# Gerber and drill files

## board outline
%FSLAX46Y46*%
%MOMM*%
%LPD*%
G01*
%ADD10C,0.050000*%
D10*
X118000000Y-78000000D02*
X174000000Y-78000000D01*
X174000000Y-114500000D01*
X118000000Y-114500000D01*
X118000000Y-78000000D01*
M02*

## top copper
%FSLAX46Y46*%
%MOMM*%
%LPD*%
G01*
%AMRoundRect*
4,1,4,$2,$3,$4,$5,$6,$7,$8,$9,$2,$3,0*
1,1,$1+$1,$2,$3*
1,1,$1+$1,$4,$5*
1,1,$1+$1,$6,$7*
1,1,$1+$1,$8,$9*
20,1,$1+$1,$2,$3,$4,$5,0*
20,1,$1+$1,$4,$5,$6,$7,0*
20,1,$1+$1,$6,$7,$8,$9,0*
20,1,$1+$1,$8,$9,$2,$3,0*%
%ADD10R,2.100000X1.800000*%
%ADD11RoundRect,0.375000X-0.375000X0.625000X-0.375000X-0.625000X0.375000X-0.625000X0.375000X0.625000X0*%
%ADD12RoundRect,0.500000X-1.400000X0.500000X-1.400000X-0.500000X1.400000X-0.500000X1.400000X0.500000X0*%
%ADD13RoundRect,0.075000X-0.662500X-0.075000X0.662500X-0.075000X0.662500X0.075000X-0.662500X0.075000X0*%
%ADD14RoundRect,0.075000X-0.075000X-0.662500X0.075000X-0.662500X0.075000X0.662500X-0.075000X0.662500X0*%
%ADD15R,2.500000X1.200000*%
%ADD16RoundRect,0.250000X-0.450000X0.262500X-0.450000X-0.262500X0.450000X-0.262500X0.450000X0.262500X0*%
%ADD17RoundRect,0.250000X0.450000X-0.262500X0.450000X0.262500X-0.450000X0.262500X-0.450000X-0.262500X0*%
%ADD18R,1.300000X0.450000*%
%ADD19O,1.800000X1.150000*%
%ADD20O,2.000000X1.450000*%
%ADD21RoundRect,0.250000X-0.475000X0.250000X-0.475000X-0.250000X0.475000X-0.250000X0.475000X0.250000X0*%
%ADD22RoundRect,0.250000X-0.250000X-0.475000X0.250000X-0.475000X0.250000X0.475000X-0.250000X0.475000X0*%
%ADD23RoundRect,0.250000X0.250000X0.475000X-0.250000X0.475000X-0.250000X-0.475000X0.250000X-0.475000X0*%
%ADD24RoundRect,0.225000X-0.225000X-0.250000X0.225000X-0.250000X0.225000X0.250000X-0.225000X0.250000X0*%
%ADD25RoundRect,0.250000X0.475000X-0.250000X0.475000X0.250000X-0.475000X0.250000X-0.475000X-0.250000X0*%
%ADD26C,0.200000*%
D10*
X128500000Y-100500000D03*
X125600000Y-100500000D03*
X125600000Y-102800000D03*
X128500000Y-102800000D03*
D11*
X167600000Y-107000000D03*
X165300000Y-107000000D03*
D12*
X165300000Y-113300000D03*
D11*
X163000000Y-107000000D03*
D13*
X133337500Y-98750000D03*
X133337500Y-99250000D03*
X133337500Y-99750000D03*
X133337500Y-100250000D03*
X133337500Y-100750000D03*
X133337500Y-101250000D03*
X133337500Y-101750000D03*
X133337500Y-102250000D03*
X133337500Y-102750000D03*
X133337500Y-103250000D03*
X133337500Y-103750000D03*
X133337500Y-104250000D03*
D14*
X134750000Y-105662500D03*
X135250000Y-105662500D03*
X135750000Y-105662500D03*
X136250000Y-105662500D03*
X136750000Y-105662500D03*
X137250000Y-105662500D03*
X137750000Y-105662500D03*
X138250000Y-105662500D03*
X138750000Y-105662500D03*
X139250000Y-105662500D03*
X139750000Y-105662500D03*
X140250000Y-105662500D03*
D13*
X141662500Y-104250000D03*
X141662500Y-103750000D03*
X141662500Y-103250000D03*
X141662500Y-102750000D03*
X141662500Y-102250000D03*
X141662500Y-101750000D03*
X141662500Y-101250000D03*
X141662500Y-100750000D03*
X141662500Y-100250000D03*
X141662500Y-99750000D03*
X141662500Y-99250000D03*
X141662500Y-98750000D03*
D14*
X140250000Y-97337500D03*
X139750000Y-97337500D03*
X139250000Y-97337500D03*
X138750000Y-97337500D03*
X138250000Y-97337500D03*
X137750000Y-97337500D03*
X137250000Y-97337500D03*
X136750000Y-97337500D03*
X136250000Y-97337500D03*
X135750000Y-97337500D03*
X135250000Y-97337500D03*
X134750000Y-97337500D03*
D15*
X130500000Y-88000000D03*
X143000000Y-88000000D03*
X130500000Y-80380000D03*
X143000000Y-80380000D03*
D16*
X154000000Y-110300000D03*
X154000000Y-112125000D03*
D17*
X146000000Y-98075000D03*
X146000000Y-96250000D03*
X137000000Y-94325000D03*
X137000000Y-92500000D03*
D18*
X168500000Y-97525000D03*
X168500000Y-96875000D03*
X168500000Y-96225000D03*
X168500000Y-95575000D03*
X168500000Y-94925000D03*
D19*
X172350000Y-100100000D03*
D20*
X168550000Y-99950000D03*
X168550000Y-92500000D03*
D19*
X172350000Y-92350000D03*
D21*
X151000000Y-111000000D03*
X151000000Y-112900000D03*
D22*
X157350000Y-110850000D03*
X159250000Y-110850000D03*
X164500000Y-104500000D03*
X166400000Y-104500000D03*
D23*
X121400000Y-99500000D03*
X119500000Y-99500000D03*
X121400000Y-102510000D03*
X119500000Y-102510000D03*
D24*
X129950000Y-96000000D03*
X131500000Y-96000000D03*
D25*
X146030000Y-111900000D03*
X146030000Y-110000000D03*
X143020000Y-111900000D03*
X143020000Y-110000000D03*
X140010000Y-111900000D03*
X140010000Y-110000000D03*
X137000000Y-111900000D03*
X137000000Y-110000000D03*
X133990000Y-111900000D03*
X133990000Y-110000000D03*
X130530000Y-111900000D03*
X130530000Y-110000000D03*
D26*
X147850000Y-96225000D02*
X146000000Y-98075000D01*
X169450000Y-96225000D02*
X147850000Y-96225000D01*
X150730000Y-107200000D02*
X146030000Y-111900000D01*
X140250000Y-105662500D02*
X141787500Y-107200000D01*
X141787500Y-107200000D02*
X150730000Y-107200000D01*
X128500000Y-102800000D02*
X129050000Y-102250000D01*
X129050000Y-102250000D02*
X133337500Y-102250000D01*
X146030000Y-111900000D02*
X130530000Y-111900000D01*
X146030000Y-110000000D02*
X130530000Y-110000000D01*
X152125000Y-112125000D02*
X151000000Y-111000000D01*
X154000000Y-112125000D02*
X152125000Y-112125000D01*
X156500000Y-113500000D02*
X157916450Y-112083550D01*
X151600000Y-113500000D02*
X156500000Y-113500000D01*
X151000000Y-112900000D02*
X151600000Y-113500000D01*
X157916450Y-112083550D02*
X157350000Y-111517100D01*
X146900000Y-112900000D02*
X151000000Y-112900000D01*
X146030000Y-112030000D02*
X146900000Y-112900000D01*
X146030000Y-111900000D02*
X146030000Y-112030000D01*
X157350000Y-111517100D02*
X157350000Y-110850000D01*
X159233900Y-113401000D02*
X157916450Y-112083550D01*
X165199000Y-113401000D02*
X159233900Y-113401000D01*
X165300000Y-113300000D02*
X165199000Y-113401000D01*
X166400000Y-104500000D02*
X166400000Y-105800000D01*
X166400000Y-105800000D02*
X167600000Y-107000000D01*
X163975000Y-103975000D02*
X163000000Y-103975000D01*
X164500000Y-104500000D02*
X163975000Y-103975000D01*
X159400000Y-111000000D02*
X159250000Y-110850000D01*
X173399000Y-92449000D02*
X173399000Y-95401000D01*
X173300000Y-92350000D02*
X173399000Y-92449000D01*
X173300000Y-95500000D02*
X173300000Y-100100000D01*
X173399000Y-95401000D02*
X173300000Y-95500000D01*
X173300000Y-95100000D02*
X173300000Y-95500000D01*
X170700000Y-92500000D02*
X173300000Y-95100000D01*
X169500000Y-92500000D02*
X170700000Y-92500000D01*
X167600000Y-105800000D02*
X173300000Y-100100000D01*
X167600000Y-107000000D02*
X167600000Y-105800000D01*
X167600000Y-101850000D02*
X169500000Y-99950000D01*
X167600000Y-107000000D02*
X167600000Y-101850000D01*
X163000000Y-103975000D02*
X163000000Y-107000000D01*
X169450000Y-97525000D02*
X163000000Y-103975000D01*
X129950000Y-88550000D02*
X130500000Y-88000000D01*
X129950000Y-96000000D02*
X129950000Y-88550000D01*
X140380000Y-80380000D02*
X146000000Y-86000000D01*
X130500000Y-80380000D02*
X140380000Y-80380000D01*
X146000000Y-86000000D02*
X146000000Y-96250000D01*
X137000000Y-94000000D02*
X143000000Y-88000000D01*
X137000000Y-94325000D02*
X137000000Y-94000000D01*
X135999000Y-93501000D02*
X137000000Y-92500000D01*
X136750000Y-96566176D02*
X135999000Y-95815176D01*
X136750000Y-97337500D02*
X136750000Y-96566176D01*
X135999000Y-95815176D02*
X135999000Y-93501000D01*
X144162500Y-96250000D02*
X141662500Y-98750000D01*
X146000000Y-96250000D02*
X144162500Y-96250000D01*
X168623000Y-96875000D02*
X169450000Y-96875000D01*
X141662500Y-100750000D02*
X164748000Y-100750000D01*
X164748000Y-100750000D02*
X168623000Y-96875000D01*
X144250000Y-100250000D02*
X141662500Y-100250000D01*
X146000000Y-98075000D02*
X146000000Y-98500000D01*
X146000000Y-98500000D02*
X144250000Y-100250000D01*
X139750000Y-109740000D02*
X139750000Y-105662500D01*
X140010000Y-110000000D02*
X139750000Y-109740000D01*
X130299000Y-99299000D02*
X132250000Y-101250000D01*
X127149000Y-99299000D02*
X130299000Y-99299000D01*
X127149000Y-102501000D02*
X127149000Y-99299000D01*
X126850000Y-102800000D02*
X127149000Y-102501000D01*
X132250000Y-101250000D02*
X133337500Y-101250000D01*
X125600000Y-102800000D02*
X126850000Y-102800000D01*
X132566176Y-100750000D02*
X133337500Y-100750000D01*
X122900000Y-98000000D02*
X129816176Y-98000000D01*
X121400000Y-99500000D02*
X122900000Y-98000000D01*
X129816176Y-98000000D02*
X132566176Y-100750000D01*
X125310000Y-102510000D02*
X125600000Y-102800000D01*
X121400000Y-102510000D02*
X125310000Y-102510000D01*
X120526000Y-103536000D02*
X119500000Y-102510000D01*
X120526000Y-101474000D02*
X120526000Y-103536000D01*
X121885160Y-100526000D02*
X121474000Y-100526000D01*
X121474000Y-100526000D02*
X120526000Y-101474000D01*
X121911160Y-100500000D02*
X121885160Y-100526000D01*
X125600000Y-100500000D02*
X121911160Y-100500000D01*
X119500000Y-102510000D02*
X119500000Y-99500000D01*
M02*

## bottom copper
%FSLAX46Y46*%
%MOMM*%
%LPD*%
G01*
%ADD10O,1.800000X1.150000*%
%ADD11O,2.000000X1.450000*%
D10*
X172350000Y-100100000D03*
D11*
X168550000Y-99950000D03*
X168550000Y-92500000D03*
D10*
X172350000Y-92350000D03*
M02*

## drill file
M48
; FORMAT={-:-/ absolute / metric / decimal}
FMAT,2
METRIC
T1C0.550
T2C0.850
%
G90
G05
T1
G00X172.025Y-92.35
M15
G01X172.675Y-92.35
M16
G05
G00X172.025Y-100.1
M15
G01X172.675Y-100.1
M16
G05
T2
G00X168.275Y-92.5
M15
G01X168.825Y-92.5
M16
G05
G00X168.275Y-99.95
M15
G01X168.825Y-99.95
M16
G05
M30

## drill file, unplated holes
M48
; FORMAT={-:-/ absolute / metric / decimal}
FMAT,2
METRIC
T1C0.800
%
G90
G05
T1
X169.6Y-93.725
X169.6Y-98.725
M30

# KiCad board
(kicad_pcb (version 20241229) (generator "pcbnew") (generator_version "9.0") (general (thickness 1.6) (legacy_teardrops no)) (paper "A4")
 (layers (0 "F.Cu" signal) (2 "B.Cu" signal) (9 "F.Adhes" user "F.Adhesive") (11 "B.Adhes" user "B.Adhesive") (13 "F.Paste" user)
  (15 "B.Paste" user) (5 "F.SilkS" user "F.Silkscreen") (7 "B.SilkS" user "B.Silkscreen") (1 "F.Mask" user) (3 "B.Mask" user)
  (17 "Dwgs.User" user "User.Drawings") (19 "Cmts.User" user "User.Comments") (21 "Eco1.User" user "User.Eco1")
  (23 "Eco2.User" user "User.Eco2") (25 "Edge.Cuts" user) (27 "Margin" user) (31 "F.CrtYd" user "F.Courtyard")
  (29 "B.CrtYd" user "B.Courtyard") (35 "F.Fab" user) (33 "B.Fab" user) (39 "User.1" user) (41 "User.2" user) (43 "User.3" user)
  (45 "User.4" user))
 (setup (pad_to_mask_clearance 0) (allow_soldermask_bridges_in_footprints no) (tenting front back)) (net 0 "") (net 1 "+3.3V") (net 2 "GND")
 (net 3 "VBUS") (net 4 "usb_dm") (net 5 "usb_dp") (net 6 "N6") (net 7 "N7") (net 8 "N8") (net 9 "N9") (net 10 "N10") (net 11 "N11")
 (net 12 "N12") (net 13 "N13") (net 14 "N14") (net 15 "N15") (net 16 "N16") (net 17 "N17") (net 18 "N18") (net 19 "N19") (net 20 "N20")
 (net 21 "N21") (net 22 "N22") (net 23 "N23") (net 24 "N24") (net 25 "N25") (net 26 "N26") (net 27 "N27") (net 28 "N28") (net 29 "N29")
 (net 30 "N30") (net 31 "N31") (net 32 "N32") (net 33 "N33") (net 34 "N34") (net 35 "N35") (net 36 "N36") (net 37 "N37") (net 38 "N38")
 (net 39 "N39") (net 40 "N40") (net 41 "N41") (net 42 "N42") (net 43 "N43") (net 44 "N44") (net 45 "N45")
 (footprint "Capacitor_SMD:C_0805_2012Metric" (layer "F.Cu") (at 133.99 110.95 90)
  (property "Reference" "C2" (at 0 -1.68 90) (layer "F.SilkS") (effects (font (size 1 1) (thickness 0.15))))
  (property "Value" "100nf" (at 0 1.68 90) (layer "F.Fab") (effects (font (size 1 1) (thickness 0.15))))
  (pad "1" smd roundrect (at -0.95 0 90) (size 1 1.45) (layers "F.Cu" "F.Mask" "F.Paste") (roundrect_rratio 0.25) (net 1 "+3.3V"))
  (pad "2" smd roundrect (at 0.95 0 90) (size 1 1.45) (layers "F.Cu" "F.Mask" "F.Paste") (roundrect_rratio 0.25) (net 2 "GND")))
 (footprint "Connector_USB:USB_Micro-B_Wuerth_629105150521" (layer "F.Cu") (at 170.4 96.225 90)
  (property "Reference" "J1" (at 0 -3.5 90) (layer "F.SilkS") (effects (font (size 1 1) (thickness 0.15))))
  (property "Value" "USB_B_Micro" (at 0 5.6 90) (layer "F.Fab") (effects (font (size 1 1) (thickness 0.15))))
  (pad "" np_thru_hole oval (at -2.5 -0.8 90) (size 0.8 0.8) (drill 0.8) (layers "*.Cu" "*.Mask"))
  (pad "" np_thru_hole oval (at 2.5 -0.8 90) (size 0.8 0.8) (drill 0.8) (layers "*.Cu" "*.Mask"))
  (pad "1" smd rect (at -1.3 -1.9 90) (size 0.45 1.3) (layers "F.Cu" "F.Mask" "F.Paste") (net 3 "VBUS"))
  (pad "2" smd rect (at -0.65 -1.9 90) (size 0.45 1.3) (layers "F.Cu" "F.Mask" "F.Paste") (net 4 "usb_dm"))
  (pad "3" smd rect (at 0 -1.9 90) (size 0.45 1.3) (layers "F.Cu" "F.Mask" "F.Paste") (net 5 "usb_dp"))
  (pad "4" smd rect (at 0.65 -1.9 90) (size 0.45 1.3) (layers "F.Cu" "F.Mask" "F.Paste") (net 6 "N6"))
  (pad "5" smd rect (at 1.3 -1.9 90) (size 0.45 1.3) (layers "F.Cu" "F.Mask" "F.Paste") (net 2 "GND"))
  (pad "6" thru_hole oval (at -3.875 1.95 90) (size 1.15 1.8) (drill oval 0.55 1.2) (layers "*.Cu" "*.Mask") (remove_unused_layers no)
   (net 2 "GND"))
  (pad "6" thru_hole oval (at -3.725 -1.85 90) (size 1.45 2) (drill oval 0.85 1.4) (layers "*.Cu" "*.Mask") (remove_unused_layers no)
   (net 2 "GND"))
  (pad "6" thru_hole oval (at 3.725 -1.85 90) (size 1.45 2) (drill oval 0.85 1.4) (layers "*.Cu" "*.Mask") (remove_unused_layers no)
   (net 2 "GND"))
  (pad "6" thru_hole oval (at 3.875 1.95 90) (size 1.15 1.8) (drill oval 0.55 1.2) (layers "*.Cu" "*.Mask") (remove_unused_layers no)
   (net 2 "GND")))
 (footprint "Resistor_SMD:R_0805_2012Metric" (layer "F.Cu") (at 137 93.4125 90)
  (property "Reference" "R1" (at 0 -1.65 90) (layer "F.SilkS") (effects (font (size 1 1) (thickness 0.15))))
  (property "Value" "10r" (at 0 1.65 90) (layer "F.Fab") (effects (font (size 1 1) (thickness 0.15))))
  (pad "1" smd roundrect (at -0.9125 0 90) (size 1.025 1.4) (layers "F.Cu" "F.Mask" "F.Paste") (roundrect_rratio 0.243902) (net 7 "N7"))
  (pad "2" smd roundrect (at 0.9125 0 90) (size 1.025 1.4) (layers "F.Cu" "F.Mask" "F.Paste") (roundrect_rratio 0.243902) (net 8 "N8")))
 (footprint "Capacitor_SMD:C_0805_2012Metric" (layer "F.Cu") (at 143.02 110.95 90)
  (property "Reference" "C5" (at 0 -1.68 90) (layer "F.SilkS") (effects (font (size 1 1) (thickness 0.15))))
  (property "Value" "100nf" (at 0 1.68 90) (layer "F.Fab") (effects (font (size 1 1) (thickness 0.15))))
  (pad "1" smd roundrect (at -0.95 0 90) (size 1 1.45) (layers "F.Cu" "F.Mask" "F.Paste") (roundrect_rratio 0.25) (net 1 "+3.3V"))
  (pad "2" smd roundrect (at 0.95 0 90) (size 1 1.45) (layers "F.Cu" "F.Mask" "F.Paste") (roundrect_rratio 0.25) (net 2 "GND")))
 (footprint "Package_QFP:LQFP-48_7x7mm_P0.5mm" (layer "F.Cu") (at 137.5 101.5)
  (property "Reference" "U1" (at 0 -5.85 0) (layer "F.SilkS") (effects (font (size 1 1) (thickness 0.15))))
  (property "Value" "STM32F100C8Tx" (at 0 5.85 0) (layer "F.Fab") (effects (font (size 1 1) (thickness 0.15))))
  (pad "1" smd roundrect (at -4.1625 -2.75) (size 1.475 0.3) (layers "F.Cu" "F.Mask" "F.Paste") (roundrect_rratio 0.25) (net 1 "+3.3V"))
  (pad "2" smd roundrect (at -4.1625 -2.25) (size 1.475 0.3) (layers "F.Cu" "F.Mask" "F.Paste") (roundrect_rratio 0.25) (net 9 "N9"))
  (pad "3" smd roundrect (at -4.1625 -1.75) (size 1.475 0.3) (layers "F.Cu" "F.Mask" "F.Paste") (roundrect_rratio 0.25) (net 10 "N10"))
  (pad "4" smd roundrect (at -4.1625 -1.25) (size 1.475 0.3) (layers "F.Cu" "F.Mask" "F.Paste") (roundrect_rratio 0.25) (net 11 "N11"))
  (pad "5" smd roundrect (at -4.1625 -0.75) (size 1.475 0.3) (layers "F.Cu" "F.Mask" "F.Paste") (roundrect_rratio 0.25) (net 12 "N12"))
  (pad "6" smd roundrect (at -4.1625 -0.25) (size 1.475 0.3) (layers "F.Cu" "F.Mask" "F.Paste") (roundrect_rratio 0.25) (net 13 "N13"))
  (pad "7" smd roundrect (at -4.1625 0.25) (size 1.475 0.3) (layers "F.Cu" "F.Mask" "F.Paste") (roundrect_rratio 0.25) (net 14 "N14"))
  (pad "8" smd roundrect (at -4.1625 0.75) (size 1.475 0.3) (layers "F.Cu" "F.Mask" "F.Paste") (roundrect_rratio 0.25) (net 2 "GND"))
  (pad "9" smd roundrect (at -4.1625 1.25) (size 1.475 0.3) (layers "F.Cu" "F.Mask" "F.Paste") (roundrect_rratio 0.25) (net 1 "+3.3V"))
  (pad "10" smd roundrect (at -4.1625 1.75) (size 1.475 0.3) (layers "F.Cu" "F.Mask" "F.Paste") (roundrect_rratio 0.25) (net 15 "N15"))
  (pad "11" smd roundrect (at -4.1625 2.25) (size 1.475 0.3) (layers "F.Cu" "F.Mask" "F.Paste") (roundrect_rratio 0.25) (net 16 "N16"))
  (pad "12" smd roundrect (at -4.1625 2.75) (size 1.475 0.3) (layers "F.Cu" "F.Mask" "F.Paste") (roundrect_rratio 0.25) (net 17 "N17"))
  (pad "13" smd roundrect (at -2.75 4.1625) (size 0.3 1.475) (layers "F.Cu" "F.Mask" "F.Paste") (roundrect_rratio 0.25) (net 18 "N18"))
  (pad "14" smd roundrect (at -2.25 4.1625) (size 0.3 1.475) (layers "F.Cu" "F.Mask" "F.Paste") (roundrect_rratio 0.25) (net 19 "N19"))
  (pad "15" smd roundrect (at -1.75 4.1625) (size 0.3 1.475) (layers "F.Cu" "F.Mask" "F.Paste") (roundrect_rratio 0.25) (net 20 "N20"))
  (pad "16" smd roundrect (at -1.25 4.1625) (size 0.3 1.475) (layers "F.Cu" "F.Mask" "F.Paste") (roundrect_rratio 0.25) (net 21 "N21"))
  (pad "17" smd roundrect (at -0.75 4.1625) (size 0.3 1.475) (layers "F.Cu" "F.Mask" "F.Paste") (roundrect_rratio 0.25) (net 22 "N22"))
  (pad "18" smd roundrect (at -0.25 4.1625) (size 0.3 1.475) (layers "F.Cu" "F.Mask" "F.Paste") (roundrect_rratio 0.25) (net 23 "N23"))
  (pad "19" smd roundrect (at 0.25 4.1625) (size 0.3 1.475) (layers "F.Cu" "F.Mask" "F.Paste") (roundrect_rratio 0.25) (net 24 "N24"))
  (pad "20" smd roundrect (at 0.75 4.1625) (size 0.3 1.475) (layers "F.Cu" "F.Mask" "F.Paste") (roundrect_rratio 0.25) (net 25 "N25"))
  (pad "21" smd roundrect (at 1.25 4.1625) (size 0.3 1.475) (layers "F.Cu" "F.Mask" "F.Paste") (roundrect_rratio 0.25) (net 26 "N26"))
  (pad "22" smd roundrect (at 1.75 4.1625) (size 0.3 1.475) (layers "F.Cu" "F.Mask" "F.Paste") (roundrect_rratio 0.25) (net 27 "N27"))
  (pad "23" smd roundrect (at 2.25 4.1625) (size 0.3 1.475) (layers "F.Cu" "F.Mask" "F.Paste") (roundrect_rratio 0.25) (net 2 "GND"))
  (pad "24" smd roundrect (at 2.75 4.1625) (size 0.3 1.475) (layers "F.Cu" "F.Mask" "F.Paste") (roundrect_rratio 0.25) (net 1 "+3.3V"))
  (pad "25" smd roundrect (at 4.1625 2.75) (size 1.475 0.3) (layers "F.Cu" "F.Mask" "F.Paste") (roundrect_rratio 0.25) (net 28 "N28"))
  (pad "26" smd roundrect (at 4.1625 2.25) (size 1.475 0.3) (layers "F.Cu" "F.Mask" "F.Paste") (roundrect_rratio 0.25) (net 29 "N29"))
  (pad "27" smd roundrect (at 4.1625 1.75) (size 1.475 0.3) (layers "F.Cu" "F.Mask" "F.Paste") (roundrect_rratio 0.25) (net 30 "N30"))
  (pad "28" smd roundrect (at 4.1625 1.25) (size 1.475 0.3) (layers "F.Cu" "F.Mask" "F.Paste") (roundrect_rratio 0.25) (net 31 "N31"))
  (pad "29" smd roundrect (at 4.1625 0.75) (size 1.475 0.3) (layers "F.Cu" "F.Mask" "F.Paste") (roundrect_rratio 0.25) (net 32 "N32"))
  (pad "30" smd roundrect (at 4.1625 0.25) (size 1.475 0.3) (layers "F.Cu" "F.Mask" "F.Paste") (roundrect_rratio 0.25) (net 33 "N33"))
  (pad "31" smd roundrect (at 4.1625 -0.25) (size 1.475 0.3) (layers "F.Cu" "F.Mask" "F.Paste") (roundrect_rratio 0.25) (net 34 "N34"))
  (pad "32" smd roundrect (at 4.1625 -0.75) (size 1.475 0.3) (layers "F.Cu" "F.Mask" "F.Paste") (roundrect_rratio 0.25) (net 4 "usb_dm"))
  (pad "33" smd roundrect (at 4.1625 -1.25) (size 1.475 0.3) (layers "F.Cu" "F.Mask" "F.Paste") (roundrect_rratio 0.25) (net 5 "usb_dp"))
  (pad "34" smd roundrect (at 4.1625 -1.75) (size 1.475 0.3) (layers "F.Cu" "F.Mask" "F.Paste") (roundrect_rratio 0.25) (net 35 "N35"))
  (pad "35" smd roundrect (at 4.1625 -2.25) (size 1.475 0.3) (layers "F.Cu" "F.Mask" "F.Paste") (roundrect_rratio 0.25) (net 2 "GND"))
  (pad "36" smd roundrect (at 4.1625 -2.75) (size 1.475 0.3) (layers "F.Cu" "F.Mask" "F.Paste") (roundrect_rratio 0.25) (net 1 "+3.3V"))
  (pad "37" smd roundrect (at 2.75 -4.1625) (size 0.3 1.475) (layers "F.Cu" "F.Mask" "F.Paste") (roundrect_rratio 0.25) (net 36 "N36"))
  (pad "38" smd roundrect (at 2.25 -4.1625) (size 0.3 1.475) (layers "F.Cu" "F.Mask" "F.Paste") (roundrect_rratio 0.25) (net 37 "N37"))
  (pad "39" smd roundrect (at 1.75 -4.1625) (size 0.3 1.475) (layers "F.Cu" "F.Mask" "F.Paste") (roundrect_rratio 0.25) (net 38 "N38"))
  (pad "40" smd roundrect (at 1.25 -4.1625) (size 0.3 1.475) (layers "F.Cu" "F.Mask" "F.Paste") (roundrect_rratio 0.25) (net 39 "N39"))
  (pad "41" smd roundrect (at 0.75 -4.1625) (size 0.3 1.475) (layers "F.Cu" "F.Mask" "F.Paste") (roundrect_rratio 0.25) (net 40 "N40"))
  (pad "42" smd roundrect (at 0.25 -4.1625) (size 0.3 1.475) (layers "F.Cu" "F.Mask" "F.Paste") (roundrect_rratio 0.25) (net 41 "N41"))
  (pad "43" smd roundrect (at -0.25 -4.1625) (size 0.3 1.475) (layers "F.Cu" "F.Mask" "F.Paste") (roundrect_rratio 0.25) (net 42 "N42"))
  (pad "44" smd roundrect (at -0.75 -4.1625) (size 0.3 1.475) (layers "F.Cu" "F.Mask" "F.Paste") (roundrect_rratio 0.25) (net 8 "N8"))
  (pad "45" smd roundrect (at -1.25 -4.1625) (size 0.3 1.475) (layers "F.Cu" "F.Mask" "F.Paste") (roundrect_rratio 0.25) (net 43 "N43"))
  (pad "46" smd roundrect (at -1.75 -4.1625) (size 0.3 1.475) (layers "F.Cu" "F.Mask" "F.Paste") (roundrect_rratio 0.25) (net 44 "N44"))
  (pad "47" smd roundrect (at -2.25 -4.1625) (size 0.3 1.475) (layers "F.Cu" "F.Mask" "F.Paste") (roundrect_rratio 0.25) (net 2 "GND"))
  (pad "48" smd roundrect (at -2.75 -4.1625) (size 0.3 1.475) (layers "F.Cu" "F.Mask" "F.Paste") (roundrect_rratio 0.25) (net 1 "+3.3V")))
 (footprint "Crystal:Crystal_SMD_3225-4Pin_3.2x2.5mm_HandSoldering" (layer "F.Cu") (at 127.05 101.65 180)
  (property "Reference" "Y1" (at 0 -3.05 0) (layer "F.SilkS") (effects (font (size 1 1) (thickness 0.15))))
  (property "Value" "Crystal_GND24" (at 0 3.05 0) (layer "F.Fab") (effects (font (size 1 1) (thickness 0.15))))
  (pad "1" smd rect (at -1.45 1.15 180) (size 2.1 1.8) (layers "F.Cu" "F.Mask" "F.Paste") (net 12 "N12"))
  (pad "2" smd rect (at 1.45 1.15 180) (size 2.1 1.8) (layers "F.Cu" "F.Mask" "F.Paste") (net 2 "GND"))
  (pad "3" smd rect (at 1.45 -1.15 180) (size 2.1 1.8) (layers "F.Cu" "F.Mask" "F.Paste") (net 13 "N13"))
  (pad "4" smd rect (at -1.45 -1.15 180) (size 2.1 1.8) (layers "F.Cu" "F.Mask" "F.Paste") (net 2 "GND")))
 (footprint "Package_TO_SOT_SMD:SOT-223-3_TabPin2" (layer "F.Cu") (at 165.3 110.15 -90)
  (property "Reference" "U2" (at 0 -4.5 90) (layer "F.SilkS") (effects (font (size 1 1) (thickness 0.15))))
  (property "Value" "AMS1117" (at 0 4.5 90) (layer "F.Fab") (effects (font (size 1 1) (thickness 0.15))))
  (pad "1" smd roundrect (at -3.15 -2.3 270) (size 2 1.5) (layers "F.Cu" "F.Mask" "F.Paste") (roundrect_rratio 0.25) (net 2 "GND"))
  (pad "2" smd roundrect (at -3.15 0 270) (size 2 1.5) (layers "F.Cu" "F.Mask" "F.Paste") (roundrect_rratio 0.25) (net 1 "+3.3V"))
  (pad "2" smd roundrect (at 3.15 0 270) (size 2 3.8) (layers "F.Cu" "F.Mask" "F.Paste") (roundrect_rratio 0.25) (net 1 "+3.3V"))
  (pad "3" smd roundrect (at -3.15 2.3 270) (size 2 1.5) (layers "F.Cu" "F.Mask" "F.Paste") (roundrect_rratio 0.25) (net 3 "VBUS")))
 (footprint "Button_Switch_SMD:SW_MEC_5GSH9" (layer "F.Cu") (at 136.75 84.19 90)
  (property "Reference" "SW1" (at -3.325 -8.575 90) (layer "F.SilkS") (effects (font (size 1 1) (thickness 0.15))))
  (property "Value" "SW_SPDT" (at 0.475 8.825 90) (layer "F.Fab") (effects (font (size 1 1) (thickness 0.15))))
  (pad "1" smd rect (at -3.81 -6.25 180) (size 2.5 1.2) (layers "F.Cu" "F.Mask" "F.Paste") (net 2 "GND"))
  (pad "2" smd rect (at -3.81 6.25 180) (size 2.5 1.2) (layers "F.Cu" "F.Mask" "F.Paste") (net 7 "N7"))
  (pad "3" smd rect (at 3.81 -6.25 180) (size 2.5 1.2) (layers "F.Cu" "F.Mask" "F.Paste") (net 1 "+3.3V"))
  (pad "4" smd rect (at 3.81 6.25 180) (size 2.5 1.2) (layers "F.Cu" "F.Mask" "F.Paste")))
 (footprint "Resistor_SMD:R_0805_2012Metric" (layer "F.Cu") (at 154 111.2125 -90)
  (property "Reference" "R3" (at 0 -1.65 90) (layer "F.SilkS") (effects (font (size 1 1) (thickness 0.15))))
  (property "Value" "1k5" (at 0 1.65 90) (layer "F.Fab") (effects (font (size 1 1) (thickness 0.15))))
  (pad "1" smd roundrect (at -0.9125 0 270) (size 1.025 1.4) (layers "F.Cu" "F.Mask" "F.Paste") (roundrect_rratio 0.243902) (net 2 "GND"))
  (pad "2" smd roundrect (at 0.9125 0 270) (size 1.025 1.4) (layers "F.Cu" "F.Mask" "F.Paste") (roundrect_rratio 0.243902) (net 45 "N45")))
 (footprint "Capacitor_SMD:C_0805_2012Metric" (layer "F.Cu") (at 140.01 110.95 90)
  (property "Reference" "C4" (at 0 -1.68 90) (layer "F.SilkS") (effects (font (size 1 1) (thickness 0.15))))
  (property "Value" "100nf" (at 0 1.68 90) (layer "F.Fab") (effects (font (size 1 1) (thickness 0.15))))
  (pad "1" smd roundrect (at -0.95 0 90) (size 1 1.45) (layers "F.Cu" "F.Mask" "F.Paste") (roundrect_rratio 0.25) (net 1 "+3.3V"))
  (pad "2" smd roundrect (at 0.95 0 90) (size 1 1.45) (layers "F.Cu" "F.Mask" "F.Paste") (roundrect_rratio 0.25) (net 2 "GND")))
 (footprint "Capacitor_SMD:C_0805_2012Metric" (layer "F.Cu") (at 120.45 102.51 180)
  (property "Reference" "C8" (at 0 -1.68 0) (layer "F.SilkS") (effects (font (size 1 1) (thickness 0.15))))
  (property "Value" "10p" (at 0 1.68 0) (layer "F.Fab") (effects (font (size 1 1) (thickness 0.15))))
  (pad "1" smd roundrect (at -0.95 0 180) (size 1 1.45) (layers "F.Cu" "F.Mask" "F.Paste") (roundrect_rratio 0.25) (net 13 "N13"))
  (pad "2" smd roundrect (at 0.95 0 180) (size 1 1.45) (layers "F.Cu" "F.Mask" "F.Paste") (roundrect_rratio 0.25) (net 2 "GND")))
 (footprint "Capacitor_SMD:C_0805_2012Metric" (layer "F.Cu") (at 151 111.95 -90)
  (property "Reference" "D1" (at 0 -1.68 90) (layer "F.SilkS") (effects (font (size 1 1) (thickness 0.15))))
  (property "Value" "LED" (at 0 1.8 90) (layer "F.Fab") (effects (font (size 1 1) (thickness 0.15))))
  (pad "1" smd roundrect (at -0.95 0 270) (size 1 1.45) (layers "F.Cu" "F.Mask" "F.Paste") (roundrect_rratio 0.25) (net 45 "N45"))
  (pad "2" smd roundrect (at 0.95 0 270) (size 1 1.45) (layers "F.Cu" "F.Mask" "F.Paste") (roundrect_rratio 0.25) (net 1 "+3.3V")))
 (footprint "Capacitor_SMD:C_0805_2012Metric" (layer "F.Cu") (at 165.45 104.5)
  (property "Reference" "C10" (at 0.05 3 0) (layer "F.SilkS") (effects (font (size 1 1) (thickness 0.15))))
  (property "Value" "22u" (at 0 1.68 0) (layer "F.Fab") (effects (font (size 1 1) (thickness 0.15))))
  (pad "1" smd roundrect (at -0.95 0) (size 1 1.45) (layers "F.Cu" "F.Mask" "F.Paste") (roundrect_rratio 0.25) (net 3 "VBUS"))
  (pad "2" smd roundrect (at 0.95 0) (size 1 1.45) (layers "F.Cu" "F.Mask" "F.Paste") (roundrect_rratio 0.25) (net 2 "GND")))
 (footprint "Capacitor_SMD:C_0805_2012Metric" (layer "F.Cu") (at 146.03 110.95 90)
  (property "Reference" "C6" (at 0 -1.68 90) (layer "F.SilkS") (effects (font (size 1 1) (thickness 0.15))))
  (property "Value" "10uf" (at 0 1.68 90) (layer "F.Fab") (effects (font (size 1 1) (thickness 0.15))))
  (pad "1" smd roundrect (at -0.95 0 90) (size 1 1.45) (layers "F.Cu" "F.Mask" "F.Paste") (roundrect_rratio 0.25) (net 1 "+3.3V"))
  (pad "2" smd roundrect (at 0.95 0 90) (size 1 1.45) (layers "F.Cu" "F.Mask" "F.Paste") (roundrect_rratio 0.25) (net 2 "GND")))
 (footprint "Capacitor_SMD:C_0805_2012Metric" (layer "F.Cu") (at 158.3 110.85)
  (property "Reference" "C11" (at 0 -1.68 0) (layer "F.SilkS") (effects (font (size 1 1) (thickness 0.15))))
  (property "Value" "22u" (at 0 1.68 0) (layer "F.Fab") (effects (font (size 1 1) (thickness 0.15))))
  (pad "1" smd roundrect (at -0.95 0) (size 1 1.45) (layers "F.Cu" "F.Mask" "F.Paste") (roundrect_rratio 0.25) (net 1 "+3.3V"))
  (pad "2" smd roundrect (at 0.95 0) (size 1 1.45) (layers "F.Cu" "F.Mask" "F.Paste") (roundrect_rratio 0.25) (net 2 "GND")))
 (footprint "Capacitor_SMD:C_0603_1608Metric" (layer "F.Cu") (at 130.725 96)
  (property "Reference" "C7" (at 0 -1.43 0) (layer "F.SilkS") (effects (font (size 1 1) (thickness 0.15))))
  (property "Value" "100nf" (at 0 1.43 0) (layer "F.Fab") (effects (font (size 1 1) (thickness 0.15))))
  (pad "1" smd roundrect (at -0.775 0) (size 0.9 0.95) (layers "F.Cu" "F.Mask" "F.Paste") (roundrect_rratio 0.25) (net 2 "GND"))
  (pad "2" smd roundrect (at 0.775 0) (size 0.9 0.95) (layers "F.Cu" "F.Mask" "F.Paste") (roundrect_rratio 0.25) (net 14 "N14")))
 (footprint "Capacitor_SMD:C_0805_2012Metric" (layer "F.Cu") (at 120.45 99.5 180)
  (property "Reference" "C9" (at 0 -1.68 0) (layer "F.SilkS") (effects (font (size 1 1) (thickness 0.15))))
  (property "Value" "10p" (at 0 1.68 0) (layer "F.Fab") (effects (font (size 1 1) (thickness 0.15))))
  (pad "1" smd roundrect (at -0.95 0 180) (size 1 1.45) (layers "F.Cu" "F.Mask" "F.Paste") (roundrect_rratio 0.25) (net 12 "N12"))
  (pad "2" smd roundrect (at 0.95 0 180) (size 1 1.45) (layers "F.Cu" "F.Mask" "F.Paste") (roundrect_rratio 0.25) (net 2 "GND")))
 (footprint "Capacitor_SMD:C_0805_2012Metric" (layer "F.Cu") (at 137 110.95 90)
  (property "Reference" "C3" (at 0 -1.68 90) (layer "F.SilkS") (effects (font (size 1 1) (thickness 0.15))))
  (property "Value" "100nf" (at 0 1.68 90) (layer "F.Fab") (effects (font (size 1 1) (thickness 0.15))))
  (pad "1" smd roundrect (at -0.95 0 90) (size 1 1.45) (layers "F.Cu" "F.Mask" "F.Paste") (roundrect_rratio 0.25) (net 1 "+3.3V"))
  (pad "2" smd roundrect (at 0.95 0 90) (size 1 1.45) (layers "F.Cu" "F.Mask" "F.Paste") (roundrect_rratio 0.25) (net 2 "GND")))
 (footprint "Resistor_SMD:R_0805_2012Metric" (layer "F.Cu") (at 146 97.1625 90)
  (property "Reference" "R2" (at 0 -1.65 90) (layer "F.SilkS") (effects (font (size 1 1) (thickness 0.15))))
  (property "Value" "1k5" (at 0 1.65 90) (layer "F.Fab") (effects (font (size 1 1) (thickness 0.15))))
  (pad "1" smd roundrect (at -0.9125 0 90) (size 1.025 1.4) (layers "F.Cu" "F.Mask" "F.Paste") (roundrect_rratio 0.243902) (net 5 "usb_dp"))
  (pad "2" smd roundrect (at 0.9125 0 90) (size 1.025 1.4) (layers "F.Cu" "F.Mask" "F.Paste") (roundrect_rratio 0.243902) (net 1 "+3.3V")))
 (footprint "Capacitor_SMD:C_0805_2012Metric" (layer "F.Cu") (at 130.53 110.95 90)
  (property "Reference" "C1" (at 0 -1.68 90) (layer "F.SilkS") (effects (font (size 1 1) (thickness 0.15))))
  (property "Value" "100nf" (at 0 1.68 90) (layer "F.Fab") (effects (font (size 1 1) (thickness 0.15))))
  (pad "1" smd roundrect (at -0.95 0 90) (size 1 1.45) (layers "F.Cu" "F.Mask" "F.Paste") (roundrect_rratio 0.25) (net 1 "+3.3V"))
  (pad "2" smd roundrect (at 0.95 0 90) (size 1 1.45) (layers "F.Cu" "F.Mask" "F.Paste") (roundrect_rratio 0.25) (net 2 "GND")))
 (gr_rect (start 118 78) (end 174 114.5) (stroke (width 0.05) (type default)) (fill no) (layer "Edge.Cuts"))
 (segment (start 121.88516 100.526) (end 121.474 100.526) (width 0.2) (layer "F.Cu") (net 2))
 (segment (start 121.91116 100.5) (end 121.88516 100.526) (width 0.2) (layer "F.Cu") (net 2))
 (segment (start 139.75 109.74) (end 139.75 105.6625) (width 0.2) (layer "F.Cu") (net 2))
 (segment (start 173.3 95.5) (end 173.3 100.1) (width 0.2) (layer "F.Cu") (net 2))
 (segment (start 146.03 110) (end 130.53 110) (width 0.2) (layer "F.Cu") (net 2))
 (segment (start 120.526 101.474) (end 120.526 103.536) (width 0.2) (layer "F.Cu") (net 2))
 (segment (start 173.399 95.401) (end 173.3 95.5) (width 0.2) (layer "F.Cu") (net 2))
 (segment (start 166.4 104.5) (end 166.4 105.8) (width 0.2) (layer "F.Cu") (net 2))
 (segment (start 128.5 102.8) (end 129.05 102.25) (width 0.2) (layer "F.Cu") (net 2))
 (segment (start 125.6 100.5) (end 121.91116 100.5) (width 0.2) (layer "F.Cu") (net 2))
 (segment (start 170.7 92.5) (end 173.3 95.1) (width 0.2) (layer "F.Cu") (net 2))
 (segment (start 167.6 107) (end 167.6 101.85) (width 0.2) (layer "F.Cu") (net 2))
 (segment (start 140.01 110) (end 139.75 109.74) (width 0.2) (layer "F.Cu") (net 2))
 (segment (start 173.3 92.35) (end 173.399 92.449) (width 0.2) (layer "F.Cu") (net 2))
 (segment (start 173.399 92.449) (end 173.399 95.401) (width 0.2) (layer "F.Cu") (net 2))
 (segment (start 120.526 103.536) (end 119.5 102.51) (width 0.2) (layer "F.Cu") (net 2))
 (segment (start 167.6 105.8) (end 173.3 100.1) (width 0.2) (layer "F.Cu") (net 2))
 (segment (start 159.4 111) (end 159.25 110.85) (width 0.2) (layer "F.Cu") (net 2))
 (segment (start 173.3 95.1) (end 173.3 95.5) (width 0.2) (layer "F.Cu") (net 2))
 (segment (start 129.05 102.25) (end 133.3375 102.25) (width 0.2) (layer "F.Cu") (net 2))
 (segment (start 167.6 107) (end 167.6 105.8) (width 0.2) (layer "F.Cu") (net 2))
 (segment (start 129.95 88.55) (end 130.5 88) (width 0.2) (layer "F.Cu") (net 2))
 (segment (start 129.95 96) (end 129.95 88.55) (width 0.2) (layer "F.Cu") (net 2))
 (segment (start 167.6 101.85) (end 169.5 99.95) (width 0.2) (layer "F.Cu") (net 2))
 (segment (start 169.5 92.5) (end 170.7 92.5) (width 0.2) (layer "F.Cu") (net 2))
 (segment (start 166.4 105.8) (end 167.6 107) (width 0.2) (layer "F.Cu") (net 2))
 (segment (start 119.5 102.51) (end 119.5 99.5) (width 0.2) (layer "F.Cu") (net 2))
 (segment (start 121.474 100.526) (end 120.526 101.474) (width 0.2) (layer "F.Cu") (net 2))
 (segment (start 141.7875 107.2) (end 150.73 107.2) (width 0.2) (layer "F.Cu") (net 1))
 (segment (start 140.38 80.38) (end 146 86) (width 0.2) (layer "F.Cu") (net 1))
 (segment (start 146 96.25) (end 144.1625 96.25) (width 0.2) (layer "F.Cu") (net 1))
 (segment (start 146.03 111.9) (end 146.03 112.03) (width 0.2) (layer "F.Cu") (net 1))
 (segment (start 146.03 111.9) (end 130.53 111.9) (width 0.2) (layer "F.Cu") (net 1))
 (segment (start 146.9 112.9) (end 151 112.9) (width 0.2) (layer "F.Cu") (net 1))
 (segment (start 165.199 113.401) (end 159.2339 113.401) (width 0.2) (layer "F.Cu") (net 1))
 (segment (start 159.2339 113.401) (end 157.91645 112.08355) (width 0.2) (layer "F.Cu") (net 1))
 (segment (start 157.91645 112.08355) (end 157.35 111.5171) (width 0.2) (layer "F.Cu") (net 1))
 (segment (start 146 86) (end 146 96.25) (width 0.2) (layer "F.Cu") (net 1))
 (segment (start 140.25 105.6625) (end 141.7875 107.2) (width 0.2) (layer "F.Cu") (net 1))
 (segment (start 165.3 113.3) (end 165.199 113.401) (width 0.2) (layer "F.Cu") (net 1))
 (segment (start 144.1625 96.25) (end 141.6625 98.75) (width 0.2) (layer "F.Cu") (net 1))
 (segment (start 151.6 113.5) (end 156.5 113.5) (width 0.2) (layer "F.Cu") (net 1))
 (segment (start 151 112.9) (end 151.6 113.5) (width 0.2) (layer "F.Cu") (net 1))
 (segment (start 150.73 107.2) (end 146.03 111.9) (width 0.2) (layer "F.Cu") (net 1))
 (segment (start 130.5 80.38) (end 140.38 80.38) (width 0.2) (layer "F.Cu") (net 1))
 (segment (start 156.5 113.5) (end 157.91645 112.08355) (width 0.2) (layer "F.Cu") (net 1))
 (segment (start 157.35 111.5171) (end 157.35 110.85) (width 0.2) (layer "F.Cu") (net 1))
 (segment (start 146.03 112.03) (end 146.9 112.9) (width 0.2) (layer "F.Cu") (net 1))
 (segment (start 130.299 99.299) (end 132.25 101.25) (width 0.2) (layer "F.Cu") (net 13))
 (segment (start 127.149 99.299) (end 130.299 99.299) (width 0.2) (layer "F.Cu") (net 13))
 (segment (start 125.31 102.51) (end 125.6 102.8) (width 0.2) (layer "F.Cu") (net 13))
 (segment (start 126.85 102.8) (end 127.149 102.501) (width 0.2) (layer "F.Cu") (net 13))
 (segment (start 121.4 102.51) (end 125.31 102.51) (width 0.2) (layer "F.Cu") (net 13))
 (segment (start 127.149 102.501) (end 127.149 99.299) (width 0.2) (layer "F.Cu") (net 13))
 (segment (start 132.25 101.25) (end 133.3375 101.25) (width 0.2) (layer "F.Cu") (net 13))
 (segment (start 125.6 102.8) (end 126.85 102.8) (width 0.2) (layer "F.Cu") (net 13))
 (segment (start 121.4 99.5) (end 122.9 98) (width 0.2) (layer "F.Cu") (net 12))
 (segment (start 129.816176 98) (end 132.566176 100.75) (width 0.2) (layer "F.Cu") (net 12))
 (segment (start 132.566176 100.75) (end 133.3375 100.75) (width 0.2) (layer "F.Cu") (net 12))
 (segment (start 122.9 98) (end 129.816176 98) (width 0.2) (layer "F.Cu") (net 12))
 (segment (start 163.975 103.975) (end 163 103.975) (width 0.2) (layer "F.Cu") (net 3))
 (segment (start 164.5 104.5) (end 163.975 103.975) (width 0.2) (layer "F.Cu") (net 3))
 (segment (start 163 103.975) (end 163 107) (width 0.2) (layer "F.Cu") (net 3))
 (segment (start 169.45 97.525) (end 163 103.975) (width 0.2) (layer "F.Cu") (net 3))
 (segment (start 154 112.125) (end 152.125 112.125) (width 0.2) (layer "F.Cu") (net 45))
 (segment (start 152.125 112.125) (end 151 111) (width 0.2) (layer "F.Cu") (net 45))
 (segment (start 147.85 96.225) (end 146 98.075) (width 0.2) (layer "F.Cu") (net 5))
 (segment (start 169.45 96.225) (end 147.85 96.225) (width 0.2) (layer "F.Cu") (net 5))
 (segment (start 146 98.075) (end 146 98.5) (width 0.2) (layer "F.Cu") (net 5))
 (segment (start 146 98.5) (end 144.25 100.25) (width 0.2) (layer "F.Cu") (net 5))
 (segment (start 144.25 100.25) (end 141.6625 100.25) (width 0.2) (layer "F.Cu") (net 5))
 (segment (start 168.623 96.875) (end 169.45 96.875) (width 0.2) (layer "F.Cu") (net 4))
 (segment (start 164.748 100.75) (end 168.623 96.875) (width 0.2) (layer "F.Cu") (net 4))
 (segment (start 141.6625 100.75) (end 164.748 100.75) (width 0.2) (layer "F.Cu") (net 4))
 (segment (start 135.999 93.501) (end 137 92.5) (width 0.2) (layer "F.Cu") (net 8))
 (segment (start 135.999 95.815176) (end 135.999 93.501) (width 0.2) (layer "F.Cu") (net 8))
 (segment (start 136.75 96.566176) (end 135.999 95.815176) (width 0.2) (layer "F.Cu") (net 8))
 (segment (start 136.75 97.3375) (end 136.75 96.566176) (width 0.2) (layer "F.Cu") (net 8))
 (segment (start 137 94) (end 143 88) (width 0.2) (layer "F.Cu") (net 7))
 (segment (start 137 94.325) (end 137 94) (width 0.2) (layer "F.Cu") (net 7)))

